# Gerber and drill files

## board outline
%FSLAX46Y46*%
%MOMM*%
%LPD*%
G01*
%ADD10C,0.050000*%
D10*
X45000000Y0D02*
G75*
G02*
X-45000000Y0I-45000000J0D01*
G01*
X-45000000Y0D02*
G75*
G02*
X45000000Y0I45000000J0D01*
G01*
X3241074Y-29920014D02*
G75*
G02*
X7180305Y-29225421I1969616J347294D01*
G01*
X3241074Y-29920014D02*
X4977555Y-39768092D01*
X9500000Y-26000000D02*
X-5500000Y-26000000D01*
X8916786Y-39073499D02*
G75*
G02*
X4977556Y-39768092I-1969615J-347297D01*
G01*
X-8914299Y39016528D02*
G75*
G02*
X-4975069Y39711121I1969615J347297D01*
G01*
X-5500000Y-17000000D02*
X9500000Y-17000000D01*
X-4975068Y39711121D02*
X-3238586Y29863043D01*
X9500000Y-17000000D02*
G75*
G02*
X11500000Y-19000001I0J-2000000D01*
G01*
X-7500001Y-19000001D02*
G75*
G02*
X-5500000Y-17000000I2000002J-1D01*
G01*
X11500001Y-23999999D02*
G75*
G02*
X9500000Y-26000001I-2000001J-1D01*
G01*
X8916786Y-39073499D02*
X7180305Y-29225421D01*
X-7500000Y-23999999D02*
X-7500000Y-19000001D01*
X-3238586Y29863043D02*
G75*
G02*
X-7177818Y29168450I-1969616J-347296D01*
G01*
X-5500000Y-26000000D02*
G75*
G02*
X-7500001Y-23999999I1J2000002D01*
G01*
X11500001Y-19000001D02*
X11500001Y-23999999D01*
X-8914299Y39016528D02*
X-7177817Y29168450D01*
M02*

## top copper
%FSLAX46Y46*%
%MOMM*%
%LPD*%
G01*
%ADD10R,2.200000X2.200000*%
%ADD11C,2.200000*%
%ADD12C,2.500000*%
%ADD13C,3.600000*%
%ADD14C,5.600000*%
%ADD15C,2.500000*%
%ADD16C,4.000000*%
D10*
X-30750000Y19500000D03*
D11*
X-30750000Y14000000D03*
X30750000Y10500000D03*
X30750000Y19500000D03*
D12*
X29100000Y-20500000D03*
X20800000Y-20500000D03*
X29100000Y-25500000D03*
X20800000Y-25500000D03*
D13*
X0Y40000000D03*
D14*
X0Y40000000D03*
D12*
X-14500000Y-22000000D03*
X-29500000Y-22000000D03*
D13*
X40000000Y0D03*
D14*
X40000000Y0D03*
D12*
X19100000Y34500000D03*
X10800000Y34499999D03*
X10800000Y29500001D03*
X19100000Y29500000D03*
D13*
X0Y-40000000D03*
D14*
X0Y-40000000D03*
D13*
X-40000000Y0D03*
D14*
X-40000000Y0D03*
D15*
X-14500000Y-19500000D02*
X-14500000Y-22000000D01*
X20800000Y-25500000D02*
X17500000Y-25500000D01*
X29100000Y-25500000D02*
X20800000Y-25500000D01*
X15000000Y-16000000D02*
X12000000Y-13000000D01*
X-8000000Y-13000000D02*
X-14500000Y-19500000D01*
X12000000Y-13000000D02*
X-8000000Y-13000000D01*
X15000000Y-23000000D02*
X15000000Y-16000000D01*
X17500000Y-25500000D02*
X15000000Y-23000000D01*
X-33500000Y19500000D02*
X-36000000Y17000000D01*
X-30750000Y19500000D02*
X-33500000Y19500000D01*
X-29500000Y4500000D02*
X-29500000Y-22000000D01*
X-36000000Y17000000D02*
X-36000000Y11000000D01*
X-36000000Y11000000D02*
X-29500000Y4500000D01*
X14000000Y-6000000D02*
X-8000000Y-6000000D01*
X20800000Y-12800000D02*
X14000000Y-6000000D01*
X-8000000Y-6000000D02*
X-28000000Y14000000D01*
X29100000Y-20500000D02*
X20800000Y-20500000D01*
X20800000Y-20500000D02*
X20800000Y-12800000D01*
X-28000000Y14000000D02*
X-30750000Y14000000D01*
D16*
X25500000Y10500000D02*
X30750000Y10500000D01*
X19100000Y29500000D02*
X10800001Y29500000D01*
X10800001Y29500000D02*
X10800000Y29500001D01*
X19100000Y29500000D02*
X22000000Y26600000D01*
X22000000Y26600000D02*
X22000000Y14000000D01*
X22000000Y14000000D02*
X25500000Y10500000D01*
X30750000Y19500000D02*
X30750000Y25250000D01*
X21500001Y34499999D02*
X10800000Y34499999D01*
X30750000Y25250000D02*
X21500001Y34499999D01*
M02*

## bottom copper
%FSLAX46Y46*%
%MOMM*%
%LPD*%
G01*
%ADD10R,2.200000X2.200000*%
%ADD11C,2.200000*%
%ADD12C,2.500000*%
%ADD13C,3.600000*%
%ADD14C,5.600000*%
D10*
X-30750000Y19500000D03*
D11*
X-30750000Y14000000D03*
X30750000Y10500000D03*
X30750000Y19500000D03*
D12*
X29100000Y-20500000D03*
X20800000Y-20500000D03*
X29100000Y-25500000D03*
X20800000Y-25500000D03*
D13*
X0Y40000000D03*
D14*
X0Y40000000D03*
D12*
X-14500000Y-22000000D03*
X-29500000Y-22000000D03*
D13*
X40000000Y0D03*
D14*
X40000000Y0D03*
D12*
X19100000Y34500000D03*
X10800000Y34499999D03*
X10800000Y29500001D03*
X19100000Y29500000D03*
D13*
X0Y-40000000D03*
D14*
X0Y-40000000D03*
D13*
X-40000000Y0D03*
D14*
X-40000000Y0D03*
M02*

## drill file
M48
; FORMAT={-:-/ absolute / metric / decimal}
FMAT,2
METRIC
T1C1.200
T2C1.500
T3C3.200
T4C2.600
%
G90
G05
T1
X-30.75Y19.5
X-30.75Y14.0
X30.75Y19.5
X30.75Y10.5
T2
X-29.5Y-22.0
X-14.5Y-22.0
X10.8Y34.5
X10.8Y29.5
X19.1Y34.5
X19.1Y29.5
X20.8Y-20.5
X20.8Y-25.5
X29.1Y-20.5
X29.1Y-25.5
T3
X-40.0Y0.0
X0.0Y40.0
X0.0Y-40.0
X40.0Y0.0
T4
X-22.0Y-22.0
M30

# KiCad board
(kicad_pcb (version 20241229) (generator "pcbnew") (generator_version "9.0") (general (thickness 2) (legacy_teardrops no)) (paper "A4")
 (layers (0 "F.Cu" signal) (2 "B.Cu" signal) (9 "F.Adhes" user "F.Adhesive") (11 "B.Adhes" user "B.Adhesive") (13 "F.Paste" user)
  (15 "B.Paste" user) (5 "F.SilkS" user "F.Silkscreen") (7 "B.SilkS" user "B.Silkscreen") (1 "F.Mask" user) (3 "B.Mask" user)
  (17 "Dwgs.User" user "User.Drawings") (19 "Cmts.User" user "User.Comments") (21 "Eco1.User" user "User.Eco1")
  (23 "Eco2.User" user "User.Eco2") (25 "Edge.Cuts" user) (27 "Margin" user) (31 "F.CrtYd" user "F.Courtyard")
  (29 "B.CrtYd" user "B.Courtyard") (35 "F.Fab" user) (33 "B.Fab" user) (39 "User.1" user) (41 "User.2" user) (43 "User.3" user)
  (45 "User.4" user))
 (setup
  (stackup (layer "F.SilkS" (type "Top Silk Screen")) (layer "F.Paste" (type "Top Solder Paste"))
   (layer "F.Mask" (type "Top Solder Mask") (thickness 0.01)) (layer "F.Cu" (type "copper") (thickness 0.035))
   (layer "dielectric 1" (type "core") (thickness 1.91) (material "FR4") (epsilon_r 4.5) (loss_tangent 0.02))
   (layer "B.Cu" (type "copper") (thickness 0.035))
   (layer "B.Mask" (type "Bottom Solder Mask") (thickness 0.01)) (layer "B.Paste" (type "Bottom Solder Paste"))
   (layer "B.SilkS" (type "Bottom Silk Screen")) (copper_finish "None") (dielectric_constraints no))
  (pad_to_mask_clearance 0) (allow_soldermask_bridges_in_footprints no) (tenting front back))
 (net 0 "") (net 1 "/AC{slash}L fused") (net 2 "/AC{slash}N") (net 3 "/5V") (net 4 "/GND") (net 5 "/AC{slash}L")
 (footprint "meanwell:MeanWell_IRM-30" (layer "F.Cu") (at 0 -4.5)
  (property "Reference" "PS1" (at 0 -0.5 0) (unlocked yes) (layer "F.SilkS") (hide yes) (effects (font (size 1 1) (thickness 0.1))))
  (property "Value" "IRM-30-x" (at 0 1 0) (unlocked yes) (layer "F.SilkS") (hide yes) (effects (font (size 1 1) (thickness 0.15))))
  (pad "1" thru_hole rect (at -30.75 -15) (size 2.2 2.2) (drill 1.2) (layers "*.Cu" "*.Mask") (remove_unused_layers no)
   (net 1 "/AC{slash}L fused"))
  (pad "2" thru_hole circle (at -30.75 -9.5) (size 2.2 2.2) (drill 1.2) (layers "*.Cu" "*.Mask") (remove_unused_layers no)
   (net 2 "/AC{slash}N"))
  (pad "3" thru_hole circle (at 30.75 -6) (size 2.2 2.2) (drill 1.2) (layers "*.Cu" "*.Mask") (remove_unused_layers no) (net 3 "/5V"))
  (pad "4" thru_hole circle (at 30.75 -15) (size 2.2 2.2) (drill 1.2) (layers "*.Cu" "*.Mask") (remove_unused_layers no) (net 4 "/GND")))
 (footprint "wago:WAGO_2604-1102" (layer "F.Cu") (at 25 23 -90)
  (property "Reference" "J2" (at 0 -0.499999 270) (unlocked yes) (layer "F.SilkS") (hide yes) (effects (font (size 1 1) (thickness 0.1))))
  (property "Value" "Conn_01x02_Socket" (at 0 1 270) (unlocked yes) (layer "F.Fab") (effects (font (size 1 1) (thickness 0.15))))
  (pad "1" thru_hole circle (at -2.5 -4.1 270) (size 2.5 2.5) (drill 1.5) (layers "*.Cu" "*.Mask") (remove_unused_layers no)
   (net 2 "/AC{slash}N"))
  (pad "1" thru_hole circle (at -2.5 4.2 270) (size 2.5 2.5) (drill 1.5) (layers "*.Cu" "*.Mask") (remove_unused_layers no)
   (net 2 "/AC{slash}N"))
  (pad "2" thru_hole circle (at 2.5 -4.1 270) (size 2.5 2.5) (drill 1.5) (layers "*.Cu" "*.Mask") (remove_unused_layers no)
   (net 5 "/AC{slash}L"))
  (pad "2" thru_hole circle (at 2.5 4.2 270) (size 2.5 2.5) (drill 1.5) (layers "*.Cu" "*.Mask") (remove_unused_layers no)
   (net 5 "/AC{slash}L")))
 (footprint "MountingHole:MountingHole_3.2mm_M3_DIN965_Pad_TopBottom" (layer "F.Cu") (at 0 -40)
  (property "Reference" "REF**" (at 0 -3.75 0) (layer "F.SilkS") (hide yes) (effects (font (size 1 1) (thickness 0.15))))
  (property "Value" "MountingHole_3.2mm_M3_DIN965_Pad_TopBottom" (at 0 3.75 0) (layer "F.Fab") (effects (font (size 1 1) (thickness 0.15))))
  (pad "1" thru_hole circle (at 0 0) (size 3.6 3.6) (drill 3.2) (layers "*.Cu" "*.Mask") (remove_unused_layers no) (zone_connect 2))
  (pad "1" connect circle (at 0 0) (size 5.6 5.6) (layers "F.Cu" "F.Mask") (zone_connect 2))
  (pad "1" connect circle (at 0 0) (size 5.6 5.6) (layers "B.Cu" "B.Mask") (zone_connect 2)))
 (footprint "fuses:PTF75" (layer "F.Cu") (at -22 22 180)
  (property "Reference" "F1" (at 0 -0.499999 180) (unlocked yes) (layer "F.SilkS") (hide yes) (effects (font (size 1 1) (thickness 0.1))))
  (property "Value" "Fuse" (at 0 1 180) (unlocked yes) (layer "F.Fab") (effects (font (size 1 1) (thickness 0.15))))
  (pad "" np_thru_hole circle (at 0 0 180) (size 1.905 1.905) (drill 2.6) (layers "*.Cu" "*.Mask"))
  (pad "1" thru_hole circle (at -7.5 0 180) (size 2.5 2.5) (drill 1.5) (layers "*.Cu" "*.Mask") (remove_unused_layers no)
   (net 5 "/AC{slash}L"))
  (pad "2" thru_hole circle (at 7.5 0 180) (size 2.5 2.5) (drill 1.5) (layers "*.Cu" "*.Mask") (remove_unused_layers no)
   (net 1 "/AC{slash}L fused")))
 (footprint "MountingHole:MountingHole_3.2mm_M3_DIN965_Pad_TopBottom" (layer "F.Cu") (at 40 0)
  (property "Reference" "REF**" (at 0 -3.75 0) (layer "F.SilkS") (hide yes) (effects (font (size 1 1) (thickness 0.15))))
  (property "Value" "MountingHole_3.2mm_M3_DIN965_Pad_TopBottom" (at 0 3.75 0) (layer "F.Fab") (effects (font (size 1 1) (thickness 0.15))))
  (pad "1" thru_hole circle (at 0 0) (size 3.6 3.6) (drill 3.2) (layers "*.Cu" "*.Mask") (remove_unused_layers no) (zone_connect 2))
  (pad "1" connect circle (at 0 0) (size 5.6 5.6) (layers "F.Cu" "F.Mask") (zone_connect 2))
  (pad "1" connect circle (at 0 0) (size 5.6 5.6) (layers "B.Cu" "B.Mask") (zone_connect 2)))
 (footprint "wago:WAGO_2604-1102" (layer "F.Cu") (at 15 -32 -90)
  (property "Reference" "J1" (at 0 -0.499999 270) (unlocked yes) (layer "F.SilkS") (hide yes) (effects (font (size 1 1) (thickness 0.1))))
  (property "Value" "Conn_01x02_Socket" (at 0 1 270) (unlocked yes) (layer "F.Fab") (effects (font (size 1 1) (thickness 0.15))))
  (pad "1" thru_hole circle (at -2.5 -4.1 270) (size 2.5 2.5) (drill 1.5) (layers "*.Cu" "*.Mask") (remove_unused_layers no) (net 4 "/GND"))
  (pad "1" thru_hole circle (at -2.499999 4.2 270) (size 2.5 2.5) (drill 1.5) (layers "*.Cu" "*.Mask") (remove_unused_layers no)
   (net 4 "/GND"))
  (pad "2" thru_hole circle (at 2.499999 4.2 270) (size 2.5 2.5) (drill 1.5) (layers "*.Cu" "*.Mask") (remove_unused_layers no)
   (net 3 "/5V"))
  (pad "2" thru_hole circle (at 2.5 -4.1 270) (size 2.5 2.5) (drill 1.5) (layers "*.Cu" "*.Mask") (remove_unused_layers no) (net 3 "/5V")))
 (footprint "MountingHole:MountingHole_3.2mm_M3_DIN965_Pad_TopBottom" (layer "F.Cu") (at 0 40)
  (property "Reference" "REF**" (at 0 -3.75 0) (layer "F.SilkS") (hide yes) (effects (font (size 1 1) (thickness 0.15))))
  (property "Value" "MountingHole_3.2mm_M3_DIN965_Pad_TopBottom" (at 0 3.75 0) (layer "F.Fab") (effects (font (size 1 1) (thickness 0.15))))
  (pad "1" thru_hole circle (at 0 0) (size 3.6 3.6) (drill 3.2) (layers "*.Cu" "*.Mask") (remove_unused_layers no) (zone_connect 2))
  (pad "1" connect circle (at 0 0) (size 5.6 5.6) (layers "F.Cu" "F.Mask") (zone_connect 2))
  (pad "1" connect circle (at 0 0) (size 5.6 5.6) (layers "B.Cu" "B.Mask") (zone_connect 2)))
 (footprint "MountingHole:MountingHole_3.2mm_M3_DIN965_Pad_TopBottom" (layer "F.Cu") (at -40 0)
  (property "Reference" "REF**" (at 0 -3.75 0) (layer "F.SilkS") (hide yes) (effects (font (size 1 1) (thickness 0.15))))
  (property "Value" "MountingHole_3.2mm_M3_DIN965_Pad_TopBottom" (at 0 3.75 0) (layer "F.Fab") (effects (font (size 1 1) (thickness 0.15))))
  (pad "1" thru_hole circle (at 0 0) (size 3.6 3.6) (drill 3.2) (layers "*.Cu" "*.Mask") (remove_unused_layers no) (zone_connect 2))
  (pad "1" connect circle (at 0 0) (size 5.6 5.6) (layers "F.Cu" "F.Mask") (zone_connect 2))
  (pad "1" connect circle (at 0 0) (size 5.6 5.6) (layers "B.Cu" "B.Mask") (zone_connect 2)))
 (gr_circle (center 0 0) (end 0 45) (stroke (width 0.05) (type default)) (fill no) (layer "Edge.Cuts"))
 (gr_arc (start 3.241074 29.920014) (mid 4.863393 27.603103) (end 7.180305 29.225421) (stroke (width 0.05) (type default))
  (layer "Edge.Cuts"))
 (gr_line (start 3.241074 29.920014) (end 4.977555 39.768092) (stroke (width 0.05) (type default)) (layer "Edge.Cuts"))
 (gr_line (start 9.5 26) (end -5.5 26) (stroke (width 0.05) (type default)) (layer "Edge.Cuts"))
 (gr_arc (start 8.916786 39.073499) (mid 7.294467 41.390411) (end 4.977555 39.768092) (stroke (width 0.05) (type default))
  (layer "Edge.Cuts"))
 (gr_arc (start -8.914299 -39.016528) (mid -7.29198 -41.33344) (end -4.975068 -39.711121) (stroke (width 0.05) (type default))
  (layer "Edge.Cuts"))
 (gr_line (start -5.5 17) (end 9.5 17) (stroke (width 0.05) (type default)) (layer "Edge.Cuts"))
 (gr_line (start -4.975068 -39.711121) (end -3.238586 -29.863043) (stroke (width 0.05) (type default)) (layer "Edge.Cuts"))
 (gr_arc (start 9.5 17) (mid 10.914214 17.585787) (end 11.500001 19.000001) (stroke (width 0.05) (type default)) (layer "Edge.Cuts"))
 (gr_arc (start -7.500001 19.000001) (mid -6.914214 17.585787) (end -5.5 17) (stroke (width 0.05) (type default)) (layer "Edge.Cuts"))
 (gr_arc (start 11.500001 23.999999) (mid 10.914214 25.414213) (end 9.5 26) (stroke (width 0.05) (type default)) (layer "Edge.Cuts"))
 (gr_line (start 8.916786 39.073499) (end 7.180305 29.225421) (stroke (width 0.05) (type default)) (layer "Edge.Cuts"))
 (gr_line (start -7.5 23.999999) (end -7.5 19.000001) (stroke (width 0.05) (type default)) (layer "Edge.Cuts"))
 (gr_arc (start -3.238586 -29.863043) (mid -4.860905 -27.546132) (end -7.177817 -29.16845) (stroke (width 0.05) (type default))
  (layer "Edge.Cuts"))
 (gr_arc (start -5.5 26) (mid -6.914214 25.414213) (end -7.500001 23.999999) (stroke (width 0.05) (type default)) (layer "Edge.Cuts"))
 (gr_line (start 11.500001 19.000001) (end 11.500001 23.999999) (stroke (width 0.05) (type default)) (layer "Edge.Cuts"))
 (gr_line (start -8.914299 -39.016528) (end -7.177817 -29.16845) (stroke (width 0.05) (type default)) (layer "Edge.Cuts"))
 (segment (start -14.5 19.5) (end -14.5 22) (width 2.5) (layer "F.Cu") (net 5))
 (segment (start 20.8 25.5) (end 17.5 25.5) (width 2.5) (layer "F.Cu") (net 5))
 (segment (start 29.1 25.5) (end 20.8 25.5) (width 2.5) (layer "F.Cu") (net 5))
 (segment (start 15 16) (end 12 13) (width 2.5) (layer "F.Cu") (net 5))
 (segment (start -8 13) (end -14.5 19.5) (width 2.5) (layer "F.Cu") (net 5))
 (segment (start 12 13) (end -8 13) (width 2.5) (layer "F.Cu") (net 5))
 (segment (start 15 23) (end 15 16) (width 2.5) (layer "F.Cu") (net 5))
 (segment (start 17.5 25.5) (end 15 23) (width 2.5) (layer "F.Cu") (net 5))
 (segment (start -33.5 -19.5) (end -36 -17) (width 2.5) (layer "F.Cu") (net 1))
 (segment (start -30.75 -19.5) (end -33.5 -19.5) (width 2.5) (layer "F.Cu") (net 1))
 (segment (start -29.5 -4.5) (end -29.5 22) (width 2.5) (layer "F.Cu") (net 1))
 (segment (start -36 -17) (end -36 -11) (width 2.5) (layer "F.Cu") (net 1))
 (segment (start -36 -11) (end -29.5 -4.5) (width 2.5) (layer "F.Cu") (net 1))
 (segment (start 14 6) (end -8 6) (width 2.5) (layer "F.Cu") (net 2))
 (segment (start 20.8 12.8) (end 14 6) (width 2.5) (layer "F.Cu") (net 2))
 (segment (start -8 6) (end -28 -14) (width 2.5) (layer "F.Cu") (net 2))
 (segment (start 29.1 20.5) (end 20.8 20.5) (width 2.5) (layer "F.Cu") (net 2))
 (segment (start 20.8 20.5) (end 20.8 12.8) (width 2.5) (layer "F.Cu") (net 2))
 (segment (start -28 -14) (end -30.75 -14) (width 2.5) (layer "F.Cu") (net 2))
 (segment (start 25.5 -10.5) (end 30.75 -10.5) (width 4) (layer "F.Cu") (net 3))
 (segment (start 19.1 -29.5) (end 10.800001 -29.5) (width 4) (layer "F.Cu") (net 3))
 (segment (start 10.800001 -29.5) (end 10.8 -29.500001) (width 4) (layer "F.Cu") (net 3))
 (segment (start 19.1 -29.5) (end 22 -26.6) (width 4) (layer "F.Cu") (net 3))
 (segment (start 22 -26.6) (end 22 -14) (width 4) (layer "F.Cu") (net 3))
 (segment (start 22 -14) (end 25.5 -10.5) (width 4) (layer "F.Cu") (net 3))
 (segment (start 30.75 -19.5) (end 30.75 -25.25) (width 4) (layer "F.Cu") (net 4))
 (segment (start 21.500001 -34.499999) (end 10.8 -34.499999) (width 4) (layer "F.Cu") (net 4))
 (segment (start 30.75 -25.25) (end 21.500001 -34.499999) (width 4) (layer "F.Cu") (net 4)))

